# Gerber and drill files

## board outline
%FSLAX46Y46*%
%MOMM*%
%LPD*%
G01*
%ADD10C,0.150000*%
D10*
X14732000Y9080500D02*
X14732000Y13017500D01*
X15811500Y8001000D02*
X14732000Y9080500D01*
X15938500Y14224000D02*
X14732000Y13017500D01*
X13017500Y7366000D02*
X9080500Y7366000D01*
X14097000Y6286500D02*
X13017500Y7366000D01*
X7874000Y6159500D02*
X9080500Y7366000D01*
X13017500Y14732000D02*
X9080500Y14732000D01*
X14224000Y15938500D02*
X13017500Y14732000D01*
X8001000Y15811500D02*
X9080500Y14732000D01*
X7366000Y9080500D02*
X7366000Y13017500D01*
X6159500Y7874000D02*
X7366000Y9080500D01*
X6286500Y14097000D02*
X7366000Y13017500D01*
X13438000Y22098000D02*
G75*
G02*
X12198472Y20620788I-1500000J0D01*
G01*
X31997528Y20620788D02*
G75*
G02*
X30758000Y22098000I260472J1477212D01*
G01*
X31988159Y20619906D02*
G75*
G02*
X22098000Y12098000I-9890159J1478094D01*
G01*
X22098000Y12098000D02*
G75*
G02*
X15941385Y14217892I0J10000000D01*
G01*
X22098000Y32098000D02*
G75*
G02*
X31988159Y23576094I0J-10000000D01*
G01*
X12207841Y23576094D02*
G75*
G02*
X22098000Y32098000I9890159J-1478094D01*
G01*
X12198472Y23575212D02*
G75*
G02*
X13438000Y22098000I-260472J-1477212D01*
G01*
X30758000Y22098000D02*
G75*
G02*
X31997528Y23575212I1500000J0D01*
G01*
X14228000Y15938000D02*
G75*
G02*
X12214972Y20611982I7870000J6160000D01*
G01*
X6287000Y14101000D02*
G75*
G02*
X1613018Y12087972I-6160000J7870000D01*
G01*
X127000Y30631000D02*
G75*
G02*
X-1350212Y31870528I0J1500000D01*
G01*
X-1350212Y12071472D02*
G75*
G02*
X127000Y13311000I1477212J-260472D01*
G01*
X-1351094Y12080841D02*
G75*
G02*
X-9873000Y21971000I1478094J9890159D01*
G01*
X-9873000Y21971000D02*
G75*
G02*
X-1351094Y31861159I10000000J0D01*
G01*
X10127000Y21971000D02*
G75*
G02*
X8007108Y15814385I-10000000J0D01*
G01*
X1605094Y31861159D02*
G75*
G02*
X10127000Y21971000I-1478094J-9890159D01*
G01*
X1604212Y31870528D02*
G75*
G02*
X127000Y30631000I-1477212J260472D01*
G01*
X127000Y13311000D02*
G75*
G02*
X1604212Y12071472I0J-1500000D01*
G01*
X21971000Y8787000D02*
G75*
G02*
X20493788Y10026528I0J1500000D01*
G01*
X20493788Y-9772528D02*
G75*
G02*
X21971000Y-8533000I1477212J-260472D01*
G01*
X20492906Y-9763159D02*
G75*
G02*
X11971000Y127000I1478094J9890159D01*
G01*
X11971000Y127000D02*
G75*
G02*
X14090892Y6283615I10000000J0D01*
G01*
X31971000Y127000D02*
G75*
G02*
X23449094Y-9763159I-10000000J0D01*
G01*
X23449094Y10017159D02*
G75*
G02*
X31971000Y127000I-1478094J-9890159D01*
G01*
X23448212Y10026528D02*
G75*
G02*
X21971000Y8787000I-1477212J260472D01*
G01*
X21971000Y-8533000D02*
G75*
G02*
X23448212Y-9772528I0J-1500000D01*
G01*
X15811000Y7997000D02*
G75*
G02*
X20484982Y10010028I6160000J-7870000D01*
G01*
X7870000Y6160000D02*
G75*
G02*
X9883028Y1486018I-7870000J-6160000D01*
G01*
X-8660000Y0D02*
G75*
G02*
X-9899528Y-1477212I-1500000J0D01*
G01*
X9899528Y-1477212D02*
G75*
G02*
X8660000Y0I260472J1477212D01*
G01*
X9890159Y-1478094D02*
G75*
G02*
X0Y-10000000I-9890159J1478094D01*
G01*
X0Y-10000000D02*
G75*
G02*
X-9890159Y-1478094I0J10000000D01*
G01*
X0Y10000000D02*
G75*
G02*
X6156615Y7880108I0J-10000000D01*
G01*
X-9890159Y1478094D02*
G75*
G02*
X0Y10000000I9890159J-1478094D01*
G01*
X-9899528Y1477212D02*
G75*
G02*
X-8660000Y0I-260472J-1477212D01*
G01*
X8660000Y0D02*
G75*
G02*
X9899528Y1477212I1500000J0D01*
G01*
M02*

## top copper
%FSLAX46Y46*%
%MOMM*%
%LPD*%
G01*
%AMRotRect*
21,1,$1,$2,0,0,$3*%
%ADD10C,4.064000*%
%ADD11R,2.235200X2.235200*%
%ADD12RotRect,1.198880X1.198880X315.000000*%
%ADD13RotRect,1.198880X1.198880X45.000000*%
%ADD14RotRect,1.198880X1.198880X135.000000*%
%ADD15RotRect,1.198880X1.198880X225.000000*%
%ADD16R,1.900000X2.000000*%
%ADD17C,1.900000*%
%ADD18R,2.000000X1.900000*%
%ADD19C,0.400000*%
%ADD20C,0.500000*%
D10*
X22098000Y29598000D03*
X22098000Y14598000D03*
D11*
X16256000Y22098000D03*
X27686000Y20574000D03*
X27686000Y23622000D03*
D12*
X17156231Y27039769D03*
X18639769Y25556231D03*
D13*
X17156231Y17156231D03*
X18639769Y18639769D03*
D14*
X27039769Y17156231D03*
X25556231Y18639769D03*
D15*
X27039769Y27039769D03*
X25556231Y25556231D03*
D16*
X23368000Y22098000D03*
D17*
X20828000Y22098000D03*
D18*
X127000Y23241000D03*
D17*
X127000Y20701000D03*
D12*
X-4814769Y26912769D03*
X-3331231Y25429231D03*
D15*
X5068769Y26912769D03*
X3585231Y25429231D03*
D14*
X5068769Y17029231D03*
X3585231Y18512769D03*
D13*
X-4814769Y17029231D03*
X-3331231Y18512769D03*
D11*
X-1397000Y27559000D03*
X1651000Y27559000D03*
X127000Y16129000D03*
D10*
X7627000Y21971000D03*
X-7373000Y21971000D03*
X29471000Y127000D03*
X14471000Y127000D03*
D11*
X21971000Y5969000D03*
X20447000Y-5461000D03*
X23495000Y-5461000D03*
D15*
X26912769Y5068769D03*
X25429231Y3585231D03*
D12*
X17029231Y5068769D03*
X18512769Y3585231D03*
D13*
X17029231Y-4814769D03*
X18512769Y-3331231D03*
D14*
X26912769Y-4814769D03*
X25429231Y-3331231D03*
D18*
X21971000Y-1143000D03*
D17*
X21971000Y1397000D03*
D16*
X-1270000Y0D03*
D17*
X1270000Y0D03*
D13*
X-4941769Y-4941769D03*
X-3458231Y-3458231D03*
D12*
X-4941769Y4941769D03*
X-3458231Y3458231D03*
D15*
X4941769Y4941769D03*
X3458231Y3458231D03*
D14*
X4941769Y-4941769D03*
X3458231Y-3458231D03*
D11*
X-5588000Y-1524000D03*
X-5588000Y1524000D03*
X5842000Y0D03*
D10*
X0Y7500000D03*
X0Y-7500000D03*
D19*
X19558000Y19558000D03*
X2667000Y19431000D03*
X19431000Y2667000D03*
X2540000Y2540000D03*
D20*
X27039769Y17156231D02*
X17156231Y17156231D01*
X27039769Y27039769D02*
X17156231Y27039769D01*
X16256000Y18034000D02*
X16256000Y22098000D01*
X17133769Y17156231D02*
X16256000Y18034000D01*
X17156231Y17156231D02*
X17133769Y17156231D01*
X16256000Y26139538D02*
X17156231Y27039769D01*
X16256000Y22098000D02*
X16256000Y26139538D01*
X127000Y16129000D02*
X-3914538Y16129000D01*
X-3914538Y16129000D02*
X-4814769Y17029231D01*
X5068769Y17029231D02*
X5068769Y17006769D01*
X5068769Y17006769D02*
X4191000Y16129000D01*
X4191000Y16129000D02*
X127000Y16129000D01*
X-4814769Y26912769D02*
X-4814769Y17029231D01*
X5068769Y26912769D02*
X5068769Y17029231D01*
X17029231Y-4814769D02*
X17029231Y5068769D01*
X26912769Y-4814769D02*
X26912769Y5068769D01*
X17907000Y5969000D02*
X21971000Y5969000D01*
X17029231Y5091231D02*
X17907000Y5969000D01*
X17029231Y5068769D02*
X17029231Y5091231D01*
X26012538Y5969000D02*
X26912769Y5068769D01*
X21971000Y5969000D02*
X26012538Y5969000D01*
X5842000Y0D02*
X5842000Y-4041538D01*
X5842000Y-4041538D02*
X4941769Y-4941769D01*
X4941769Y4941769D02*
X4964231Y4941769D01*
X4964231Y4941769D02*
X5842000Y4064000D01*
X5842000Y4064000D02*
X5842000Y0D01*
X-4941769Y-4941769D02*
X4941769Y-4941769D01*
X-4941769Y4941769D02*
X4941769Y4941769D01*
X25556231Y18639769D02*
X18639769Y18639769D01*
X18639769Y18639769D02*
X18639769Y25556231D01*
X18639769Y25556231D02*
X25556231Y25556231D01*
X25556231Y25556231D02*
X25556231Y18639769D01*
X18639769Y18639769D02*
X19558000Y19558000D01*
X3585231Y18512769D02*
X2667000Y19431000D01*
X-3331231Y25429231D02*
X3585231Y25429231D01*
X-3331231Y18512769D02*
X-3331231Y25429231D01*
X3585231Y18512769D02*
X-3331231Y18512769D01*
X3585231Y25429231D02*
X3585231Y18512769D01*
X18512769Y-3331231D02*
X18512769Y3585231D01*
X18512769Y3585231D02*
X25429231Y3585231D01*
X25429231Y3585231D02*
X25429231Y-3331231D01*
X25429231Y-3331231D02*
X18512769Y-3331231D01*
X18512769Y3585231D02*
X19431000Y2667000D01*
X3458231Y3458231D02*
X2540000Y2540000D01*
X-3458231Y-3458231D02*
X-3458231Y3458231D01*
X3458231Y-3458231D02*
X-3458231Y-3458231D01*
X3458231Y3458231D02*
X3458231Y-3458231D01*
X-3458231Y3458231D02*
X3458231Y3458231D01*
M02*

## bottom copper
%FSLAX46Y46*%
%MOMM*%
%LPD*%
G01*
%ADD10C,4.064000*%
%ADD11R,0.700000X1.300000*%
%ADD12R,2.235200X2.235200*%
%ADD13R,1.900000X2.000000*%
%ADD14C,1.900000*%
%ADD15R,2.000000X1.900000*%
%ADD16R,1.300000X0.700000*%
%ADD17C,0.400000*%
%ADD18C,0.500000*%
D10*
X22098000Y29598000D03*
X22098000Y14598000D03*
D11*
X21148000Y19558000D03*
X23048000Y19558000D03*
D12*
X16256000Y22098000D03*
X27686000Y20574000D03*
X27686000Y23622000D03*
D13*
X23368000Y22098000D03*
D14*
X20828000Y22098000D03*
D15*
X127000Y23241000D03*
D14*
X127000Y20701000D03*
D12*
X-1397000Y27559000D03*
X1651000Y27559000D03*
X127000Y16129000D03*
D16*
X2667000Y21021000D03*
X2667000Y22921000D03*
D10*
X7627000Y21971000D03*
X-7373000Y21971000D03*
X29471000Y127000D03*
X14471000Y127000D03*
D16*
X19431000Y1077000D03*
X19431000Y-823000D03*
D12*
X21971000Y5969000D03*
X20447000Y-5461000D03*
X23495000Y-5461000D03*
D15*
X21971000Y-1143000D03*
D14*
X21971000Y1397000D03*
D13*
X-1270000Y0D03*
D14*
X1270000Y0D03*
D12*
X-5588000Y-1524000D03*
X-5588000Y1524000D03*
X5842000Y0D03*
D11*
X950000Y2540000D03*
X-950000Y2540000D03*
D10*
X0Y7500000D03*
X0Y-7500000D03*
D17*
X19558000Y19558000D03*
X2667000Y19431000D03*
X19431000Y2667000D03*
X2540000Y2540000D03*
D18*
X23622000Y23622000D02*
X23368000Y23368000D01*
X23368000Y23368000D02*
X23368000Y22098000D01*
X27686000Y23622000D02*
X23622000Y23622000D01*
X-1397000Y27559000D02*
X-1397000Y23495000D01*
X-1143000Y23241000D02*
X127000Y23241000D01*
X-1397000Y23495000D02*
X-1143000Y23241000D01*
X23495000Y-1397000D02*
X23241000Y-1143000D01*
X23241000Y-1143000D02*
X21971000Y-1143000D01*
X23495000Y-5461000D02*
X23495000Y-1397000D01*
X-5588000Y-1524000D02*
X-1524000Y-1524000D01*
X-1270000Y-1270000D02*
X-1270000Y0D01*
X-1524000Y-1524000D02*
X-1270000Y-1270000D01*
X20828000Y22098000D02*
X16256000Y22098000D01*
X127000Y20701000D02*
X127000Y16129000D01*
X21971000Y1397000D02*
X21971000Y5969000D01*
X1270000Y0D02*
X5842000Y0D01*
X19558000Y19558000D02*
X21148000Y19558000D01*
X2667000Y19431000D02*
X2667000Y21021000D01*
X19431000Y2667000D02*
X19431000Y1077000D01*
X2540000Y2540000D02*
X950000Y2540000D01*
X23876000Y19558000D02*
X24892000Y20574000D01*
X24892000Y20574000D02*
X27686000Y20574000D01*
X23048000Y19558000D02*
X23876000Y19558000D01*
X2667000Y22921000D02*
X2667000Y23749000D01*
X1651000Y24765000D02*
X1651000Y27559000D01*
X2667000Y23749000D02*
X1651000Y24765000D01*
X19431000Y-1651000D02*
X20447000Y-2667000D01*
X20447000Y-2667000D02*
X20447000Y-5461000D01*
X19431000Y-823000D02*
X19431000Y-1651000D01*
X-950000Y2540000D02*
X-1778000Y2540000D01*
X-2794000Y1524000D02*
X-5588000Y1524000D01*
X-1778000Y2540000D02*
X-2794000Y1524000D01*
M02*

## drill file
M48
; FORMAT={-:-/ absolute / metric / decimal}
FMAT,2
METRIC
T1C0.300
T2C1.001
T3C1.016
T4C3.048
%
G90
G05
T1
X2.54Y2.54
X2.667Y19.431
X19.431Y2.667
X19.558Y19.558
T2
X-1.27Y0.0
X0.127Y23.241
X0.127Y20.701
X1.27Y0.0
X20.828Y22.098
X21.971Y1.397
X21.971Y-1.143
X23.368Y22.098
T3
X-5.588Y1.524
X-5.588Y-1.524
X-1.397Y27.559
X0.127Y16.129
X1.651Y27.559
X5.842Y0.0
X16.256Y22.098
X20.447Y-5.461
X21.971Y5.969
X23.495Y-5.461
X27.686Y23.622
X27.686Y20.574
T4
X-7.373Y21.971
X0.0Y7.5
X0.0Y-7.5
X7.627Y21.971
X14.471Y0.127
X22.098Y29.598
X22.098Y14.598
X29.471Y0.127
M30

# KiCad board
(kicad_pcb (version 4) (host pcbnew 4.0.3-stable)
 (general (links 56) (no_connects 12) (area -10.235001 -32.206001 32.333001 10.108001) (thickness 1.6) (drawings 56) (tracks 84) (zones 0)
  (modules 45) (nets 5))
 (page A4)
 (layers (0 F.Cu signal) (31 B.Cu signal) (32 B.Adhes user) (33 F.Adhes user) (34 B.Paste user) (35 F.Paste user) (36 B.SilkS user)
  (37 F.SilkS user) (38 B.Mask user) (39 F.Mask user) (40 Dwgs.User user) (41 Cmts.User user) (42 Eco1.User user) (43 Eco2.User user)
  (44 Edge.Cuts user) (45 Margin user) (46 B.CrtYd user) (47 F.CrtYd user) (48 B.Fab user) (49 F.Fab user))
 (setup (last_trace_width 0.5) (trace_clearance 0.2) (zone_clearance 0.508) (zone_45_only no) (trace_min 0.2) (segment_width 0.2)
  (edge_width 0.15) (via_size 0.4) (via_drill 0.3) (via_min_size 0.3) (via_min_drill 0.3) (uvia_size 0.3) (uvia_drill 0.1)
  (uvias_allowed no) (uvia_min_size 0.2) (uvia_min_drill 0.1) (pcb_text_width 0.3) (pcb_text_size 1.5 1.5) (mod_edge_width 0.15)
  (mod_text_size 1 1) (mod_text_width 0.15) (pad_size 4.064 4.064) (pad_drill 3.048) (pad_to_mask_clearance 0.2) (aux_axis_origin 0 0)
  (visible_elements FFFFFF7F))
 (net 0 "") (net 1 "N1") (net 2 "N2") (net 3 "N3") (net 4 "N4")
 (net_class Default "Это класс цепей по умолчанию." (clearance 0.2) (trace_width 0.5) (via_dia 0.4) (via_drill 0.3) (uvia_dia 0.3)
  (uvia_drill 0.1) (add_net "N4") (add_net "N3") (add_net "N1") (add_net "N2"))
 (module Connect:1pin (layer F.Cu) (at 22.098 -29.598 180)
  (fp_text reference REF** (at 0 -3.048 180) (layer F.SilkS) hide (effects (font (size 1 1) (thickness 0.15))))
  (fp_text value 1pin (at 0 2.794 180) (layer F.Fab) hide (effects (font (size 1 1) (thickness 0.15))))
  (pad 1 thru_hole circle (at 0 0 180) (size 4.064 4.064) (drill 3.048) (layers *.Cu *.Mask F.SilkS)))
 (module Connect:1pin (layer F.Cu) (at 22.098 -14.598 180)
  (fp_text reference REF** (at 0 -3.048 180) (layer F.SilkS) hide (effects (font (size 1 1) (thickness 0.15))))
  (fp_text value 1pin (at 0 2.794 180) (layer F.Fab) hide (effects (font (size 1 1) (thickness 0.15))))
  (pad 1 thru_hole circle (at 0 0 180) (size 4.064 4.064) (drill 3.048) (layers *.Cu *.Mask F.SilkS)))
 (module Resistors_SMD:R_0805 (layer B.Cu) (at 22.098 -19.558)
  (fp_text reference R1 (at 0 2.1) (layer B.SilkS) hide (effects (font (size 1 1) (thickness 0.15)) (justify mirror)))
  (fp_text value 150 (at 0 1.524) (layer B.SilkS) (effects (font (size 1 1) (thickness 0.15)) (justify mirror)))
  (pad 1 smd rect (at -0.95 0) (size 0.7 1.3) (layers B.Cu B.Paste B.Mask) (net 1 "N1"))
  (pad 2 smd rect (at 0.95 0) (size 0.7 1.3) (layers B.Cu B.Paste B.Mask) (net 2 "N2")))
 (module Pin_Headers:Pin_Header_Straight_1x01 (layer B.Cu) (at 16.256 -22.098 180)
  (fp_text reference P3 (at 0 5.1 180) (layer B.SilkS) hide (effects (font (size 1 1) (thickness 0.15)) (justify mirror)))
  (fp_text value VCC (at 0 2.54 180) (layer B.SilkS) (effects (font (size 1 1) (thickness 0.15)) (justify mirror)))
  (pad 1 thru_hole rect (at 0 0 180) (size 2.2352 2.2352) (drill 1.016) (layers *.Cu *.Mask B.SilkS) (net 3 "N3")))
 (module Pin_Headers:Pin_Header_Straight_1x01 (layer B.Cu) (at 27.686 -20.574 180)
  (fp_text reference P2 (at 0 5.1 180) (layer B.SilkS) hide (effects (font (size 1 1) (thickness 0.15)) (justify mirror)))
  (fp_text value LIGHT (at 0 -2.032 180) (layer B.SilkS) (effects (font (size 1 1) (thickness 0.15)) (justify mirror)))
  (pad 1 thru_hole rect (at 0 0 180) (size 2.2352 2.2352) (drill 1.016) (layers *.Cu *.Mask B.SilkS) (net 2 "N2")))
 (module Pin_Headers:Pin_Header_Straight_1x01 (layer B.Cu) (at 27.686 -23.622 180)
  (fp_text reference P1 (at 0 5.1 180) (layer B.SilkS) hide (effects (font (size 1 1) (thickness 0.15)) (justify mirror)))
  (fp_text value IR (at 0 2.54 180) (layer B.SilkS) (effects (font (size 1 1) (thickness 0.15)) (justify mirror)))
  (pad 1 thru_hole rect (at 0 0 180) (size 2.2352 2.2352) (drill 1.016) (layers *.Cu *.Mask B.SilkS) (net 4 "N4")))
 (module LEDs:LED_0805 (layer F.Cu) (at 17.898 -26.298 135)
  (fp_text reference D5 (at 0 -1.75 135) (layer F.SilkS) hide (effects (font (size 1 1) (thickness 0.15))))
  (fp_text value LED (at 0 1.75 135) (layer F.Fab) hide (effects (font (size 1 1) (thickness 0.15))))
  (pad 2 smd rect (at 1.04902 0 315) (size 1.19888 1.19888) (layers F.Cu F.Paste F.Mask) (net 3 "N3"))
  (pad 1 smd rect (at -1.04902 0 315) (size 1.19888 1.19888) (layers F.Cu F.Paste F.Mask) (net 1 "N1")))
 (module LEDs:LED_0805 (layer F.Cu) (at 17.898 -17.898 225)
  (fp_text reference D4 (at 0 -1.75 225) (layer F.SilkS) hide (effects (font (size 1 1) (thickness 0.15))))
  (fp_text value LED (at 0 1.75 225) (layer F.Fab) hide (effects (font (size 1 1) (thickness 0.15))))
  (pad 2 smd rect (at 1.04902 0 45) (size 1.19888 1.19888) (layers F.Cu F.Paste F.Mask) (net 3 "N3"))
  (pad 1 smd rect (at -1.04902 0 45) (size 1.19888 1.19888) (layers F.Cu F.Paste F.Mask) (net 1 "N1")))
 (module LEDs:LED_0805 (layer F.Cu) (at 26.298 -17.898 315)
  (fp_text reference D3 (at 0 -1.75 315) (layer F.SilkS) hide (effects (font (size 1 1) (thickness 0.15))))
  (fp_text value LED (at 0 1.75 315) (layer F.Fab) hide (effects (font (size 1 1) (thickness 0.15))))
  (pad 2 smd rect (at 1.04902 0 135) (size 1.19888 1.19888) (layers F.Cu F.Paste F.Mask) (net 3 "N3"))
  (pad 1 smd rect (at -1.04902 0 135) (size 1.19888 1.19888) (layers F.Cu F.Paste F.Mask) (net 1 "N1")))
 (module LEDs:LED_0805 (layer F.Cu) (at 26.298 -26.298 45)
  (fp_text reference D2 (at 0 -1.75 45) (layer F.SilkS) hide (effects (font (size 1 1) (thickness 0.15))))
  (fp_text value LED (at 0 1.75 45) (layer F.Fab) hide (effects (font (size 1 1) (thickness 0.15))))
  (pad 2 smd rect (at 1.04902 0 225) (size 1.19888 1.19888) (layers F.Cu F.Paste F.Mask) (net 3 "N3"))
  (pad 1 smd rect (at -1.04902 0 225) (size 1.19888 1.19888) (layers F.Cu F.Paste F.Mask) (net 1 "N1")))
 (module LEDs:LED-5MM (layer F.Cu) (at 23.368 -22.098 180)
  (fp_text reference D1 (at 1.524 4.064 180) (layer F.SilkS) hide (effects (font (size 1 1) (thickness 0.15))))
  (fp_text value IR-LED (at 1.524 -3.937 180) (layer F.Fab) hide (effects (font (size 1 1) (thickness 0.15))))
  (pad 1 thru_hole rect (at 0 0 270) (size 2 1.9) (drill 1.00076) (layers *.Cu *.Mask F.SilkS) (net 4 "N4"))
  (pad 2 thru_hole circle (at 2.54 0 180) (size 1.9 1.9) (drill 1.00076) (layers *.Cu *.Mask F.SilkS) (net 3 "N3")))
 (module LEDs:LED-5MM (layer F.Cu) (at 0.127 -23.241 270)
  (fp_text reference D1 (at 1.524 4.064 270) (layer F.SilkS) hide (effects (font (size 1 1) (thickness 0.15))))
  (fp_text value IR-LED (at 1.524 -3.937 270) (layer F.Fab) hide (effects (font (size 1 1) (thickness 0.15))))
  (pad 1 thru_hole rect (at 0 0) (size 2 1.9) (drill 1.00076) (layers *.Cu *.Mask F.SilkS) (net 4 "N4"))
  (pad 2 thru_hole circle (at 2.54 0 270) (size 1.9 1.9) (drill 1.00076) (layers *.Cu *.Mask F.SilkS) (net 3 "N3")))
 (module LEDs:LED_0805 (layer F.Cu) (at -4.073 -26.171 135)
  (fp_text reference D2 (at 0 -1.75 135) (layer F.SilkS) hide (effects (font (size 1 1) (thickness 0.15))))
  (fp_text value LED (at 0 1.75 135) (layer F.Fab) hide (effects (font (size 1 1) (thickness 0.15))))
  (pad 2 smd rect (at 1.04902 0 315) (size 1.19888 1.19888) (layers F.Cu F.Paste F.Mask) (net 3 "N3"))
  (pad 1 smd rect (at -1.04902 0 315) (size 1.19888 1.19888) (layers F.Cu F.Paste F.Mask) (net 1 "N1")))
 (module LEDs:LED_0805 (layer F.Cu) (at 4.327 -26.171 45)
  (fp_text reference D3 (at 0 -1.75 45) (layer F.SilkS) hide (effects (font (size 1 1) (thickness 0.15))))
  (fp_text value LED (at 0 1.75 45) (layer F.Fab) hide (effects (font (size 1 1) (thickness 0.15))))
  (pad 2 smd rect (at 1.04902 0 225) (size 1.19888 1.19888) (layers F.Cu F.Paste F.Mask) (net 3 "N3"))
  (pad 1 smd rect (at -1.04902 0 225) (size 1.19888 1.19888) (layers F.Cu F.Paste F.Mask) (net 1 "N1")))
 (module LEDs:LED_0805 (layer F.Cu) (at 4.327 -17.771 315)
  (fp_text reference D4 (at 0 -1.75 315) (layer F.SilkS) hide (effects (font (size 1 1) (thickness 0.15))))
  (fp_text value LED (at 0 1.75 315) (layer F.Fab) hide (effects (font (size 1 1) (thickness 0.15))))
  (pad 2 smd rect (at 1.04902 0 135) (size 1.19888 1.19888) (layers F.Cu F.Paste F.Mask) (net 3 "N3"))
  (pad 1 smd rect (at -1.04902 0 135) (size 1.19888 1.19888) (layers F.Cu F.Paste F.Mask) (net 1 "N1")))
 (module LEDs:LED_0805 (layer F.Cu) (at -4.073 -17.771 225)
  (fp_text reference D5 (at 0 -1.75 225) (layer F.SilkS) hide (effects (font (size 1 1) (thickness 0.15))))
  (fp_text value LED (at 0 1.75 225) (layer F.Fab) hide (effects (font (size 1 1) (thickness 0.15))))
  (pad 2 smd rect (at 1.04902 0 45) (size 1.19888 1.19888) (layers F.Cu F.Paste F.Mask) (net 3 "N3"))
  (pad 1 smd rect (at -1.04902 0 45) (size 1.19888 1.19888) (layers F.Cu F.Paste F.Mask) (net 1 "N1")))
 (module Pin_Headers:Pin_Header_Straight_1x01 (layer B.Cu) (at -1.397 -27.559 270)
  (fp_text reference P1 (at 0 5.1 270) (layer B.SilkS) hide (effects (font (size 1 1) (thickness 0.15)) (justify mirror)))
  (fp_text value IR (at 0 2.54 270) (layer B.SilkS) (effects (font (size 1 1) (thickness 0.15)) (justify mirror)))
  (pad 1 thru_hole rect (at 0 0 270) (size 2.2352 2.2352) (drill 1.016) (layers *.Cu *.Mask B.SilkS) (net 4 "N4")))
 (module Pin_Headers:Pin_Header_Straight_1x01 (layer B.Cu) (at 1.651 -27.559 270)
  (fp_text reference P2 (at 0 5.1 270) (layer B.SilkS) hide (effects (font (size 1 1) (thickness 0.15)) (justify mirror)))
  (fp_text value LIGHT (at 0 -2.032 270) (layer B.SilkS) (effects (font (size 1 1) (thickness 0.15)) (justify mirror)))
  (pad 1 thru_hole rect (at 0 0 270) (size 2.2352 2.2352) (drill 1.016) (layers *.Cu *.Mask B.SilkS) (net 2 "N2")))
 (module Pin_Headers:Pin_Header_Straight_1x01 (layer B.Cu) (at 0.127 -16.129 270)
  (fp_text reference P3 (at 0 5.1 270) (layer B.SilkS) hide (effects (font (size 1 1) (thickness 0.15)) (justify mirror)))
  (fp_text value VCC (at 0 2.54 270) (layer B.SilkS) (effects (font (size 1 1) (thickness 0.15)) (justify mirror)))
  (pad 1 thru_hole rect (at 0 0 270) (size 2.2352 2.2352) (drill 1.016) (layers *.Cu *.Mask B.SilkS) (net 3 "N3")))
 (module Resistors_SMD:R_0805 (layer B.Cu) (at 2.667 -21.971 90)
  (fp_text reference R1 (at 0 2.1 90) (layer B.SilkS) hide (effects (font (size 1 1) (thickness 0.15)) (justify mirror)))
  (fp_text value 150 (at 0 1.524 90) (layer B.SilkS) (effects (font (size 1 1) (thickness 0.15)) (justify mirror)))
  (pad 1 smd rect (at -0.95 0 90) (size 0.7 1.3) (layers B.Cu B.Paste B.Mask) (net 1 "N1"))
  (pad 2 smd rect (at 0.95 0 90) (size 0.7 1.3) (layers B.Cu B.Paste B.Mask) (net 2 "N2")))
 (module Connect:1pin (layer F.Cu) (at 7.627 -21.971 270)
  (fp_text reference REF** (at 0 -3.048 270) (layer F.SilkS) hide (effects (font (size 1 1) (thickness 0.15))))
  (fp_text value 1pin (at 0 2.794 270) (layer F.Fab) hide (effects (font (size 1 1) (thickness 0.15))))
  (pad 1 thru_hole circle (at 0 0 270) (size 4.064 4.064) (drill 3.048) (layers *.Cu *.Mask F.SilkS)))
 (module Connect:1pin (layer F.Cu) (at -7.373 -21.971 270)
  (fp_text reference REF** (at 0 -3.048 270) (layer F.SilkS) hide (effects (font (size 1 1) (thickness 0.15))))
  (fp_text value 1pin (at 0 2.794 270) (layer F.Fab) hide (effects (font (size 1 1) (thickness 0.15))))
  (pad 1 thru_hole circle (at 0 0 270) (size 4.064 4.064) (drill 3.048) (layers *.Cu *.Mask F.SilkS)))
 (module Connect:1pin (layer F.Cu) (at 29.471 -0.127 90)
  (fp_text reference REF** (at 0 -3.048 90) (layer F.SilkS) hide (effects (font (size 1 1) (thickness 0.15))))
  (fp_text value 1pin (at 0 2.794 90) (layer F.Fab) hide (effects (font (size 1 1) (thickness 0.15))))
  (pad 1 thru_hole circle (at 0 0 90) (size 4.064 4.064) (drill 3.048) (layers *.Cu *.Mask F.SilkS)))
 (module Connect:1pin (layer F.Cu) (at 14.471 -0.127 90)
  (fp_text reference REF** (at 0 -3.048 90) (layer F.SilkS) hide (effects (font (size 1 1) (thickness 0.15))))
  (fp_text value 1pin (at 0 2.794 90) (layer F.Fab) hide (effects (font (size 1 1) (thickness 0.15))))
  (pad 1 thru_hole circle (at 0 0 90) (size 4.064 4.064) (drill 3.048) (layers *.Cu *.Mask F.SilkS)))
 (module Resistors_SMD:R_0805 (layer B.Cu) (at 19.431 -0.127 270)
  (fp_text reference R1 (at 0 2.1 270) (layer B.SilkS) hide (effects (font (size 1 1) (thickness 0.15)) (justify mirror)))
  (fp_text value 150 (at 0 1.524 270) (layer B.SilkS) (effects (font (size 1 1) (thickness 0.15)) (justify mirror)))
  (pad 1 smd rect (at -0.95 0 270) (size 0.7 1.3) (layers B.Cu B.Paste B.Mask) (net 1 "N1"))
  (pad 2 smd rect (at 0.95 0 270) (size 0.7 1.3) (layers B.Cu B.Paste B.Mask) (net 2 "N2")))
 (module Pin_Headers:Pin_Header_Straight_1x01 (layer B.Cu) (at 21.971 -5.969 90)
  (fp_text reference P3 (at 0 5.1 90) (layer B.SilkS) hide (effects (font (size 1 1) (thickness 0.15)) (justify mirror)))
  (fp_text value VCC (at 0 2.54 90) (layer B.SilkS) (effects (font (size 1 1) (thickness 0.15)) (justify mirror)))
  (pad 1 thru_hole rect (at 0 0 90) (size 2.2352 2.2352) (drill 1.016) (layers *.Cu *.Mask B.SilkS) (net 3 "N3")))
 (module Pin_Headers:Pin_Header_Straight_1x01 (layer B.Cu) (at 20.447 5.461 90)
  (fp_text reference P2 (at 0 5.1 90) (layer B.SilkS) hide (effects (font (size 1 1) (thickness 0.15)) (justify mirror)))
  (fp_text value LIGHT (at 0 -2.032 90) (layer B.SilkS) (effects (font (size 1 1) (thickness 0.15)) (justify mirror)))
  (pad 1 thru_hole rect (at 0 0 90) (size 2.2352 2.2352) (drill 1.016) (layers *.Cu *.Mask B.SilkS) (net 2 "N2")))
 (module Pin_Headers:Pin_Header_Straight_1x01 (layer B.Cu) (at 23.495 5.461 90)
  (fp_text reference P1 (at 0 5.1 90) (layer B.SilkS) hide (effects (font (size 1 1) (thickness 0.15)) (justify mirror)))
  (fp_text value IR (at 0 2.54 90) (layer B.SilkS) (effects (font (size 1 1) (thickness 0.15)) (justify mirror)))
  (pad 1 thru_hole rect (at 0 0 90) (size 2.2352 2.2352) (drill 1.016) (layers *.Cu *.Mask B.SilkS) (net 4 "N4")))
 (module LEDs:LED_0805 (layer F.Cu) (at 26.171 -4.327 45)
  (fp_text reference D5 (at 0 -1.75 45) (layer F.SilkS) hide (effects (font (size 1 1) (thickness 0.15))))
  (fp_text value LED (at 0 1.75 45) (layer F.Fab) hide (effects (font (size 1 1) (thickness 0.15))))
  (pad 2 smd rect (at 1.04902 0 225) (size 1.19888 1.19888) (layers F.Cu F.Paste F.Mask) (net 3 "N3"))
  (pad 1 smd rect (at -1.04902 0 225) (size 1.19888 1.19888) (layers F.Cu F.Paste F.Mask) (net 1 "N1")))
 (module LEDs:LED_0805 (layer F.Cu) (at 17.771 -4.327 135)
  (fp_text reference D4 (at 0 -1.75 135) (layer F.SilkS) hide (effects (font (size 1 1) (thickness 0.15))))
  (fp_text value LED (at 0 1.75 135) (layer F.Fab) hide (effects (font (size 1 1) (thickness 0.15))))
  (pad 2 smd rect (at 1.04902 0 315) (size 1.19888 1.19888) (layers F.Cu F.Paste F.Mask) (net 3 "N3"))
  (pad 1 smd rect (at -1.04902 0 315) (size 1.19888 1.19888) (layers F.Cu F.Paste F.Mask) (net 1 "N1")))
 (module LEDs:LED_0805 (layer F.Cu) (at 17.771 4.073 225)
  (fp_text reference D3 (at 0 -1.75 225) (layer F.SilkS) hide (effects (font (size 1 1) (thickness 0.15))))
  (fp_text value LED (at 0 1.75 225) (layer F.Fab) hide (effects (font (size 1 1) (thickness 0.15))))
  (pad 2 smd rect (at 1.04902 0 45) (size 1.19888 1.19888) (layers F.Cu F.Paste F.Mask) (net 3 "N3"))
  (pad 1 smd rect (at -1.04902 0 45) (size 1.19888 1.19888) (layers F.Cu F.Paste F.Mask) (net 1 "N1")))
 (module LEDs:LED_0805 (layer F.Cu) (at 26.171 4.073 315)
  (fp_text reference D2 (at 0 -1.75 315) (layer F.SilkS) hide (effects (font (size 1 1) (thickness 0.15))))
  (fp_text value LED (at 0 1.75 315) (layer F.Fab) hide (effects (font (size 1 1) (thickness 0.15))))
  (pad 2 smd rect (at 1.04902 0 135) (size 1.19888 1.19888) (layers F.Cu F.Paste F.Mask) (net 3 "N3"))
  (pad 1 smd rect (at -1.04902 0 135) (size 1.19888 1.19888) (layers F.Cu F.Paste F.Mask) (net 1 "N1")))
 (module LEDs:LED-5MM (layer F.Cu) (at 21.971 1.143 90)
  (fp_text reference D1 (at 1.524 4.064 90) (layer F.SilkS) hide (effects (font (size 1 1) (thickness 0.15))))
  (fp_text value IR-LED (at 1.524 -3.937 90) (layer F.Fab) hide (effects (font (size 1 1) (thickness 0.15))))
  (pad 1 thru_hole rect (at 0 0 180) (size 2 1.9) (drill 1.00076) (layers *.Cu *.Mask F.SilkS) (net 4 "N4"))
  (pad 2 thru_hole circle (at 2.54 0 90) (size 1.9 1.9) (drill 1.00076) (layers *.Cu *.Mask F.SilkS) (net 3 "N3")))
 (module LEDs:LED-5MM (layer F.Cu) (at -1.27 0)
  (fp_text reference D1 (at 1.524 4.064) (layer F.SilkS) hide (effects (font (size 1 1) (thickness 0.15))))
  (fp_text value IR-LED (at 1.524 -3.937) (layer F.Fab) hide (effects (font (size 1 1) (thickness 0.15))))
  (pad 1 thru_hole rect (at 0 0 90) (size 2 1.9) (drill 1.00076) (layers *.Cu *.Mask F.SilkS) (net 4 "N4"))
  (pad 2 thru_hole circle (at 2.54 0) (size 1.9 1.9) (drill 1.00076) (layers *.Cu *.Mask F.SilkS) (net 3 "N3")))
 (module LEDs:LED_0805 (layer F.Cu) (at -4.2 4.2 225)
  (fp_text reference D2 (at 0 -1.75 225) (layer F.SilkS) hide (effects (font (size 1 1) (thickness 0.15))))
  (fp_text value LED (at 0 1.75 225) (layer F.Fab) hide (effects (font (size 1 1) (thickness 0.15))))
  (pad 2 smd rect (at 1.04902 0 45) (size 1.19888 1.19888) (layers F.Cu F.Paste F.Mask) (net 3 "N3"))
  (pad 1 smd rect (at -1.04902 0 45) (size 1.19888 1.19888) (layers F.Cu F.Paste F.Mask) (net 1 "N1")))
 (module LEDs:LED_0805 (layer F.Cu) (at -4.2 -4.2 135)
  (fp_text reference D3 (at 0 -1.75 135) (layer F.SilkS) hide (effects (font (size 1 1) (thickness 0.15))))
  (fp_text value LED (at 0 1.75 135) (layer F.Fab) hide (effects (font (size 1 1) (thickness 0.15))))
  (pad 2 smd rect (at 1.04902 0 315) (size 1.19888 1.19888) (layers F.Cu F.Paste F.Mask) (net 3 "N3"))
  (pad 1 smd rect (at -1.04902 0 315) (size 1.19888 1.19888) (layers F.Cu F.Paste F.Mask) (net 1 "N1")))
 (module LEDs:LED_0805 (layer F.Cu) (at 4.2 -4.2 45)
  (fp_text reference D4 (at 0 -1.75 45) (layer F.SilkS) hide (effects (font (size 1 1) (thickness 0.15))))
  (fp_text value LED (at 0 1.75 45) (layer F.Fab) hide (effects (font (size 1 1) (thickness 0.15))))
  (pad 2 smd rect (at 1.04902 0 225) (size 1.19888 1.19888) (layers F.Cu F.Paste F.Mask) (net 3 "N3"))
  (pad 1 smd rect (at -1.04902 0 225) (size 1.19888 1.19888) (layers F.Cu F.Paste F.Mask) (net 1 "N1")))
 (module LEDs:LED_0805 (layer F.Cu) (at 4.2 4.2 315)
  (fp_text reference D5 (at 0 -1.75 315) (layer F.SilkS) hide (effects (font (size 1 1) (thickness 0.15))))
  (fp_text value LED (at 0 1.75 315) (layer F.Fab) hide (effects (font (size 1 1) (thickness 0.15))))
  (pad 2 smd rect (at 1.04902 0 135) (size 1.19888 1.19888) (layers F.Cu F.Paste F.Mask) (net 3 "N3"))
  (pad 1 smd rect (at -1.04902 0 135) (size 1.19888 1.19888) (layers F.Cu F.Paste F.Mask) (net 1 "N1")))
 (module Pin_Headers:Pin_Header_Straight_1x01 (layer B.Cu) (at -5.588 1.524)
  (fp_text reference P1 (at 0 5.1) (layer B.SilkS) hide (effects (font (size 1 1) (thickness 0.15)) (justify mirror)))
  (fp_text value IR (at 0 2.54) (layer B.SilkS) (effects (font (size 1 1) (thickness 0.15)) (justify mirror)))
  (pad 1 thru_hole rect (at 0 0) (size 2.2352 2.2352) (drill 1.016) (layers *.Cu *.Mask B.SilkS) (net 4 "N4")))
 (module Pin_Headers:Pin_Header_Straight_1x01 (layer B.Cu) (at -5.588 -1.524)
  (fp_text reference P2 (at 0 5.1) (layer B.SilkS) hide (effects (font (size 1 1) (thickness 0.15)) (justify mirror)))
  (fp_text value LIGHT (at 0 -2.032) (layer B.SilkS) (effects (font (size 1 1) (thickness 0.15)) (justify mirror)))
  (pad 1 thru_hole rect (at 0 0) (size 2.2352 2.2352) (drill 1.016) (layers *.Cu *.Mask B.SilkS) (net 2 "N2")))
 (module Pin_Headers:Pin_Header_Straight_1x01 (layer B.Cu) (at 5.842 0)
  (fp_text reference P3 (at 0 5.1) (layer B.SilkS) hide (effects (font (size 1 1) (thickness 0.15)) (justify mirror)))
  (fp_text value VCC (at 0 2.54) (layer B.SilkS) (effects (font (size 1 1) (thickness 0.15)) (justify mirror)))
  (pad 1 thru_hole rect (at 0 0) (size 2.2352 2.2352) (drill 1.016) (layers *.Cu *.Mask B.SilkS) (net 3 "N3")))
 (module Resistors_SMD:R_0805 (layer B.Cu) (at 0 -2.54 180)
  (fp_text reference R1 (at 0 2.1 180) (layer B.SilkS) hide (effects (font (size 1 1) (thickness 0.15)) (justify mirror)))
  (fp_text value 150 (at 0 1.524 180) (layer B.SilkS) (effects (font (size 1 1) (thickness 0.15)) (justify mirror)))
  (pad 1 smd rect (at -0.95 0 180) (size 0.7 1.3) (layers B.Cu B.Paste B.Mask) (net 1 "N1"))
  (pad 2 smd rect (at 0.95 0 180) (size 0.7 1.3) (layers B.Cu B.Paste B.Mask) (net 2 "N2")))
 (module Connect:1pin (layer F.Cu) (at 0 -7.5)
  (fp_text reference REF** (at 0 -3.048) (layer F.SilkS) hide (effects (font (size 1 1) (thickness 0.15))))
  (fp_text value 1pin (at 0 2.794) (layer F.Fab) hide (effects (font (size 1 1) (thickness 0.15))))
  (pad 1 thru_hole circle (at 0 0) (size 4.064 4.064) (drill 3.048) (layers *.Cu *.Mask F.SilkS)))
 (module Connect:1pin (layer F.Cu) (at 0 7.5)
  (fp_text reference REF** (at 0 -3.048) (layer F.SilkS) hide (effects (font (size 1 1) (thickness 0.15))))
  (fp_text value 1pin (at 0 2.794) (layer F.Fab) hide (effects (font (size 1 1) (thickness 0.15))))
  (pad 1 thru_hole circle (at 0 0) (size 4.064 4.064) (drill 3.048) (layers *.Cu *.Mask F.SilkS)))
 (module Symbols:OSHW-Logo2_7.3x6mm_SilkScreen (layer F.Cu) (at 11.049 -11.2395)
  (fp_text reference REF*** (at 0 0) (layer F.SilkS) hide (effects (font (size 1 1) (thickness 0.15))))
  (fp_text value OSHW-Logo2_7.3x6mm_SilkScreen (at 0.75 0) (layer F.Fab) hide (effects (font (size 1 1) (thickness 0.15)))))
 (gr_line (start 14.732 -9.0805) (end 14.732 -13.0175) (angle 90) (layer Edge.Cuts) (width 0.15))
 (gr_line (start 15.8115 -8.001) (end 14.732 -9.0805) (angle 90) (layer Edge.Cuts) (width 0.15))
 (gr_line (start 15.9385 -14.224) (end 14.732 -13.0175) (angle 90) (layer Edge.Cuts) (width 0.15))
 (gr_line (start 13.0175 -7.366) (end 9.0805 -7.366) (angle 90) (layer Edge.Cuts) (width 0.15))
 (gr_line (start 14.097 -6.2865) (end 13.0175 -7.366) (angle 90) (layer Edge.Cuts) (width 0.15))
 (gr_line (start 7.874 -6.1595) (end 9.0805 -7.366) (angle 90) (layer Edge.Cuts) (width 0.15))
 (gr_line (start 13.0175 -14.732) (end 9.0805 -14.732) (angle 90) (layer Edge.Cuts) (width 0.15))
 (gr_line (start 14.224 -15.9385) (end 13.0175 -14.732) (angle 90) (layer Edge.Cuts) (width 0.15))
 (gr_line (start 8.001 -15.8115) (end 9.0805 -14.732) (angle 90) (layer Edge.Cuts) (width 0.15))
 (gr_line (start 7.366 -9.0805) (end 7.366 -13.0175) (angle 90) (layer Edge.Cuts) (width 0.15))
 (gr_line (start 6.1595 -7.874) (end 7.366 -9.0805) (angle 90) (layer Edge.Cuts) (width 0.15))
 (gr_line (start 6.2865 -14.097) (end 7.366 -13.0175) (angle 90) (layer Edge.Cuts) (width 0.15))
 (gr_arc (start 11.938 -22.098) (end 13.438 -22.098) (angle 80) (layer Edge.Cuts) (width 0.15))
 (gr_arc (start 32.258 -22.098) (end 30.758 -22.098) (angle -80) (layer Edge.Cuts) (width 0.15))
 (gr_arc (start 22.098 -22.098) (end 22.098 -12.098) (angle -81.5) (layer Edge.Cuts) (width 0.15))
 (gr_arc (start 22.098 -22.098) (end 22.098 -12.098) (angle 38) (layer Edge.Cuts) (width 0.15))
 (gr_arc (start 22.098 -22.098) (end 22.098 -32.098) (angle 81.5) (layer Edge.Cuts) (width 0.15))
 (gr_arc (start 22.098 -22.098) (end 22.098 -32.098) (angle -81.5) (layer Edge.Cuts) (width 0.15))
 (gr_arc (start 11.938 -22.098) (end 13.438 -22.098) (angle -80) (layer Edge.Cuts) (width 0.15))
 (gr_arc (start 32.258 -22.098) (end 30.758 -22.098) (angle 80) (layer Edge.Cuts) (width 0.15))
 (gr_arc (start 22.098 -22.098) (end 14.228 -15.938) (angle 29.5) (layer Edge.Cuts) (width 0.15))
 (gr_arc (start 0.127 -21.971) (end 6.287 -14.101) (angle 29.5) (layer Edge.Cuts) (width 0.15))
 (gr_arc (start 0.127 -32.131) (end 0.127 -30.631) (angle 80) (layer Edge.Cuts) (width 0.15))
 (gr_arc (start 0.127 -11.811) (end 0.127 -13.311) (angle -80) (layer Edge.Cuts) (width 0.15))
 (gr_arc (start 0.127 -21.971) (end -9.873 -21.971) (angle -81.5) (layer Edge.Cuts) (width 0.15))
 (gr_arc (start 0.127 -21.971) (end -9.873 -21.971) (angle 81.5) (layer Edge.Cuts) (width 0.15))
 (gr_arc (start 0.127 -21.971) (end 10.127 -21.971) (angle 38) (layer Edge.Cuts) (width 0.15))
 (gr_arc (start 0.127 -21.971) (end 10.127 -21.971) (angle -81.5) (layer Edge.Cuts) (width 0.15))
 (gr_arc (start 0.127 -32.131) (end 0.127 -30.631) (angle -80) (layer Edge.Cuts) (width 0.15))
 (gr_arc (start 0.127 -11.811) (end 0.127 -13.311) (angle 80) (layer Edge.Cuts) (width 0.15))
 (gr_arc (start 21.971 -10.287) (end 21.971 -8.787) (angle 80) (layer Edge.Cuts) (width 0.15))
 (gr_arc (start 21.971 10.033) (end 21.971 8.533) (angle -80) (layer Edge.Cuts) (width 0.15))
 (gr_arc (start 21.971 -0.127) (end 11.971 -0.127) (angle -81.5) (layer Edge.Cuts) (width 0.15))
 (gr_arc (start 21.971 -0.127) (end 11.971 -0.127) (angle 38) (layer Edge.Cuts) (width 0.15))
 (gr_arc (start 21.971 -0.127) (end 31.971 -0.127) (angle 81.5) (layer Edge.Cuts) (width 0.15))
 (gr_arc (start 21.971 -0.127) (end 31.971 -0.127) (angle -81.5) (layer Edge.Cuts) (width 0.15))
 (gr_arc (start 21.971 -10.287) (end 21.971 -8.787) (angle -80) (layer Edge.Cuts) (width 0.15))
 (gr_arc (start 21.971 10.033) (end 21.971 8.533) (angle 80) (layer Edge.Cuts) (width 0.15))
 (gr_arc (start 21.971 -0.127) (end 15.811 -7.997) (angle 29.5) (layer Edge.Cuts) (width 0.15))
 (gr_arc (start 0 0) (end 7.87 -6.16) (angle 29.5) (layer Edge.Cuts) (width 0.15))
 (gr_arc (start -10.16 0) (end -8.66 0) (angle 80) (layer Edge.Cuts) (width 0.15))
 (gr_arc (start 10.16 0) (end 8.66 0) (angle -80) (layer Edge.Cuts) (width 0.15))
 (gr_arc (start 0 0) (end 0 10) (angle -81.5) (layer Edge.Cuts) (width 0.15))
 (gr_arc (start 0 0) (end 0 10) (angle 81.5) (layer Edge.Cuts) (width 0.15))
 (gr_arc (start 0 0) (end 0 -10) (angle 38) (layer Edge.Cuts) (width 0.15))
 (gr_arc (start 0 0) (end 0 -10) (angle -81.5) (layer Edge.Cuts) (width 0.15))
 (gr_arc (start -10.16 0) (end -8.66 0) (angle -80) (layer Edge.Cuts) (width 0.15))
 (gr_arc (start 10.16 0) (end 8.66 0) (angle 80) (layer Edge.Cuts) (width 0.15))
 (segment (start 23.622 -23.622) (end 23.368 -23.368) (width 0.5) (layer B.Cu) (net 4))
 (segment (start 23.368 -23.368) (end 23.368 -22.098) (width 0.5) (layer B.Cu) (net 4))
 (segment (start 27.686 -23.622) (end 23.622 -23.622) (width 0.5) (layer B.Cu) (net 4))
 (segment (start -1.397 -27.559) (end -1.397 -23.495) (width 0.5) (layer B.Cu) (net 4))
 (segment (start -1.143 -23.241) (end 0.127 -23.241) (width 0.5) (layer B.Cu) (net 4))
 (segment (start -1.397 -23.495) (end -1.143 -23.241) (width 0.5) (layer B.Cu) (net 4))
 (segment (start 23.495 1.397) (end 23.241 1.143) (width 0.5) (layer B.Cu) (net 4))
 (segment (start 23.241 1.143) (end 21.971 1.143) (width 0.5) (layer B.Cu) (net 4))
 (segment (start 23.495 5.461) (end 23.495 1.397) (width 0.5) (layer B.Cu) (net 4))
 (segment (start -5.588 1.524) (end -1.524 1.524) (width 0.5) (layer B.Cu) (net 4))
 (segment (start -1.27 1.27) (end -1.27 0) (width 0.5) (layer B.Cu) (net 4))
 (segment (start -1.524 1.524) (end -1.27 1.27) (width 0.5) (layer B.Cu) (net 4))
 (segment (start 27.039769 -17.156231) (end 17.156231 -17.156231) (width 0.5) (layer F.Cu) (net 3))
 (segment (start 27.039769 -27.039769) (end 17.156231 -27.039769) (width 0.5) (layer F.Cu) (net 3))
 (segment (start 16.256 -18.034) (end 16.256 -22.098) (width 0.5) (layer F.Cu) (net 3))
 (segment (start 17.133769 -17.156231) (end 16.256 -18.034) (width 0.5) (layer F.Cu) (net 3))
 (segment (start 17.156231 -17.156231) (end 17.133769 -17.156231) (width 0.5) (layer F.Cu) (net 3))
 (segment (start 16.256 -26.139538) (end 17.156231 -27.039769) (width 0.5) (layer F.Cu) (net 3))
 (segment (start 16.256 -22.098) (end 16.256 -26.139538) (width 0.5) (layer F.Cu) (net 3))
 (segment (start 20.828 -22.098) (end 16.256 -22.098) (width 0.5) (layer B.Cu) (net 3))
 (segment (start 0.127 -20.701) (end 0.127 -16.129) (width 0.5) (layer B.Cu) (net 3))
 (segment (start 0.127 -16.129) (end -3.914538 -16.129) (width 0.5) (layer F.Cu) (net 3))
 (segment (start -3.914538 -16.129) (end -4.814769 -17.029231) (width 0.5) (layer F.Cu) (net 3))
 (segment (start 5.068769 -17.029231) (end 5.068769 -17.006769) (width 0.5) (layer F.Cu) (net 3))
 (segment (start 5.068769 -17.006769) (end 4.191 -16.129) (width 0.5) (layer F.Cu) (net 3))
 (segment (start 4.191 -16.129) (end 0.127 -16.129) (width 0.5) (layer F.Cu) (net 3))
 (segment (start -4.814769 -26.912769) (end -4.814769 -17.029231) (width 0.5) (layer F.Cu) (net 3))
 (segment (start 5.068769 -26.912769) (end 5.068769 -17.029231) (width 0.5) (layer F.Cu) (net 3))
 (segment (start 17.029231 4.814769) (end 17.029231 -5.068769) (width 0.5) (layer F.Cu) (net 3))
 (segment (start 26.912769 4.814769) (end 26.912769 -5.068769) (width 0.5) (layer F.Cu) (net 3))
 (segment (start 17.907 -5.969) (end 21.971 -5.969) (width 0.5) (layer F.Cu) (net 3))
 (segment (start 17.029231 -5.091231) (end 17.907 -5.969) (width 0.5) (layer F.Cu) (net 3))
 (segment (start 17.029231 -5.068769) (end 17.029231 -5.091231) (width 0.5) (layer F.Cu) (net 3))
 (segment (start 26.012538 -5.969) (end 26.912769 -5.068769) (width 0.5) (layer F.Cu) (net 3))
 (segment (start 21.971 -5.969) (end 26.012538 -5.969) (width 0.5) (layer F.Cu) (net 3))
 (segment (start 21.971 -1.397) (end 21.971 -5.969) (width 0.5) (layer B.Cu) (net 3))
 (segment (start 1.27 0) (end 5.842 0) (width 0.5) (layer B.Cu) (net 3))
 (segment (start 5.842 0) (end 5.842 4.041538) (width 0.5) (layer F.Cu) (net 3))
 (segment (start 5.842 4.041538) (end 4.941769 4.941769) (width 0.5) (layer F.Cu) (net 3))
 (segment (start 4.941769 -4.941769) (end 4.964231 -4.941769) (width 0.5) (layer F.Cu) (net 3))
 (segment (start 4.964231 -4.941769) (end 5.842 -4.064) (width 0.5) (layer F.Cu) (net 3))
 (segment (start 5.842 -4.064) (end 5.842 0) (width 0.5) (layer F.Cu) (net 3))
 (segment (start -4.941769 4.941769) (end 4.941769 4.941769) (width 0.5) (layer F.Cu) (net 3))
 (segment (start -4.941769 -4.941769) (end 4.941769 -4.941769) (width 0.5) (layer F.Cu) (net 3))
 (segment (start 25.556231 -18.639769) (end 18.639769 -18.639769) (width 0.5) (layer F.Cu) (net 1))
 (segment (start 18.639769 -18.639769) (end 18.639769 -25.556231) (width 0.5) (layer F.Cu) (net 1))
 (segment (start 18.639769 -25.556231) (end 25.556231 -25.556231) (width 0.5) (layer F.Cu) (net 1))
 (segment (start 25.556231 -25.556231) (end 25.556231 -18.639769) (width 0.5) (layer F.Cu) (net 1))
 (via (at 19.558 -19.558) (size 0.4) (drill 0.3) (layers F.Cu B.Cu) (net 1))
 (segment (start 19.558 -19.558) (end 21.148 -19.558) (width 0.5) (layer B.Cu) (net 1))
 (segment (start 18.639769 -18.639769) (end 19.558 -19.558) (width 0.5) (layer F.Cu) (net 1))
 (segment (start 3.585231 -18.512769) (end 2.667 -19.431) (width 0.5) (layer F.Cu) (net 1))
 (segment (start 2.667 -19.431) (end 2.667 -21.021) (width 0.5) (layer B.Cu) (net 1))
 (via (at 2.667 -19.431) (size 0.4) (drill 0.3) (layers F.Cu B.Cu) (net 1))
 (segment (start -3.331231 -25.429231) (end 3.585231 -25.429231) (width 0.5) (layer F.Cu) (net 1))
 (segment (start -3.331231 -18.512769) (end -3.331231 -25.429231) (width 0.5) (layer F.Cu) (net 1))
 (segment (start 3.585231 -18.512769) (end -3.331231 -18.512769) (width 0.5) (layer F.Cu) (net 1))
 (segment (start 3.585231 -25.429231) (end 3.585231 -18.512769) (width 0.5) (layer F.Cu) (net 1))
 (segment (start 18.512769 3.331231) (end 18.512769 -3.585231) (width 0.5) (layer F.Cu) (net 1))
 (segment (start 18.512769 -3.585231) (end 25.429231 -3.585231) (width 0.5) (layer F.Cu) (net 1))
 (segment (start 25.429231 -3.585231) (end 25.429231 3.331231) (width 0.5) (layer F.Cu) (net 1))
 (segment (start 25.429231 3.331231) (end 18.512769 3.331231) (width 0.5) (layer F.Cu) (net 1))
 (via (at 19.431 -2.667) (size 0.4) (drill 0.3) (layers F.Cu B.Cu) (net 1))
 (segment (start 19.431 -2.667) (end 19.431 -1.077) (width 0.5) (layer B.Cu) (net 1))
 (segment (start 18.512769 -3.585231) (end 19.431 -2.667) (width 0.5) (layer F.Cu) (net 1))
 (segment (start 3.458231 -3.458231) (end 2.54 -2.54) (width 0.5) (layer F.Cu) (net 1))
 (segment (start 2.54 -2.54) (end 0.95 -2.54) (width 0.5) (layer B.Cu) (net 1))
 (via (at 2.54 -2.54) (size 0.4) (drill 0.3) (layers F.Cu B.Cu) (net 1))
 (segment (start -3.458231 3.458231) (end -3.458231 -3.458231) (width 0.5) (layer F.Cu) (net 1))
 (segment (start 3.458231 3.458231) (end -3.458231 3.458231) (width 0.5) (layer F.Cu) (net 1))
 (segment (start 3.458231 -3.458231) (end 3.458231 3.458231) (width 0.5) (layer F.Cu) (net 1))
 (segment (start -3.458231 -3.458231) (end 3.458231 -3.458231) (width 0.5) (layer F.Cu) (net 1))
 (segment (start 23.876 -19.558) (end 24.892 -20.574) (width 0.5) (layer B.Cu) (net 2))
 (segment (start 24.892 -20.574) (end 27.686 -20.574) (width 0.5) (layer B.Cu) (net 2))
 (segment (start 23.048 -19.558) (end 23.876 -19.558) (width 0.5) (layer B.Cu) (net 2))
 (segment (start 2.667 -22.921) (end 2.667 -23.749) (width 0.5) (layer B.Cu) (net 2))
 (segment (start 1.651 -24.765) (end 1.651 -27.559) (width 0.5) (layer B.Cu) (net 2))
 (segment (start 2.667 -23.749) (end 1.651 -24.765) (width 0.5) (layer B.Cu) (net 2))
 (segment (start 19.431 1.651) (end 20.447 2.667) (width 0.5) (layer B.Cu) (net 2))
 (segment (start 20.447 2.667) (end 20.447 5.461) (width 0.5) (layer B.Cu) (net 2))
 (segment (start 19.431 0.823) (end 19.431 1.651) (width 0.5) (layer B.Cu) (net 2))
 (segment (start -0.95 -2.54) (end -1.778 -2.54) (width 0.5) (layer B.Cu) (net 2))
 (segment (start -2.794 -1.524) (end -5.588 -1.524) (width 0.5) (layer B.Cu) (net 2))
 (segment (start -1.778 -2.54) (end -2.794 -1.524) (width 0.5) (layer B.Cu) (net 2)))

